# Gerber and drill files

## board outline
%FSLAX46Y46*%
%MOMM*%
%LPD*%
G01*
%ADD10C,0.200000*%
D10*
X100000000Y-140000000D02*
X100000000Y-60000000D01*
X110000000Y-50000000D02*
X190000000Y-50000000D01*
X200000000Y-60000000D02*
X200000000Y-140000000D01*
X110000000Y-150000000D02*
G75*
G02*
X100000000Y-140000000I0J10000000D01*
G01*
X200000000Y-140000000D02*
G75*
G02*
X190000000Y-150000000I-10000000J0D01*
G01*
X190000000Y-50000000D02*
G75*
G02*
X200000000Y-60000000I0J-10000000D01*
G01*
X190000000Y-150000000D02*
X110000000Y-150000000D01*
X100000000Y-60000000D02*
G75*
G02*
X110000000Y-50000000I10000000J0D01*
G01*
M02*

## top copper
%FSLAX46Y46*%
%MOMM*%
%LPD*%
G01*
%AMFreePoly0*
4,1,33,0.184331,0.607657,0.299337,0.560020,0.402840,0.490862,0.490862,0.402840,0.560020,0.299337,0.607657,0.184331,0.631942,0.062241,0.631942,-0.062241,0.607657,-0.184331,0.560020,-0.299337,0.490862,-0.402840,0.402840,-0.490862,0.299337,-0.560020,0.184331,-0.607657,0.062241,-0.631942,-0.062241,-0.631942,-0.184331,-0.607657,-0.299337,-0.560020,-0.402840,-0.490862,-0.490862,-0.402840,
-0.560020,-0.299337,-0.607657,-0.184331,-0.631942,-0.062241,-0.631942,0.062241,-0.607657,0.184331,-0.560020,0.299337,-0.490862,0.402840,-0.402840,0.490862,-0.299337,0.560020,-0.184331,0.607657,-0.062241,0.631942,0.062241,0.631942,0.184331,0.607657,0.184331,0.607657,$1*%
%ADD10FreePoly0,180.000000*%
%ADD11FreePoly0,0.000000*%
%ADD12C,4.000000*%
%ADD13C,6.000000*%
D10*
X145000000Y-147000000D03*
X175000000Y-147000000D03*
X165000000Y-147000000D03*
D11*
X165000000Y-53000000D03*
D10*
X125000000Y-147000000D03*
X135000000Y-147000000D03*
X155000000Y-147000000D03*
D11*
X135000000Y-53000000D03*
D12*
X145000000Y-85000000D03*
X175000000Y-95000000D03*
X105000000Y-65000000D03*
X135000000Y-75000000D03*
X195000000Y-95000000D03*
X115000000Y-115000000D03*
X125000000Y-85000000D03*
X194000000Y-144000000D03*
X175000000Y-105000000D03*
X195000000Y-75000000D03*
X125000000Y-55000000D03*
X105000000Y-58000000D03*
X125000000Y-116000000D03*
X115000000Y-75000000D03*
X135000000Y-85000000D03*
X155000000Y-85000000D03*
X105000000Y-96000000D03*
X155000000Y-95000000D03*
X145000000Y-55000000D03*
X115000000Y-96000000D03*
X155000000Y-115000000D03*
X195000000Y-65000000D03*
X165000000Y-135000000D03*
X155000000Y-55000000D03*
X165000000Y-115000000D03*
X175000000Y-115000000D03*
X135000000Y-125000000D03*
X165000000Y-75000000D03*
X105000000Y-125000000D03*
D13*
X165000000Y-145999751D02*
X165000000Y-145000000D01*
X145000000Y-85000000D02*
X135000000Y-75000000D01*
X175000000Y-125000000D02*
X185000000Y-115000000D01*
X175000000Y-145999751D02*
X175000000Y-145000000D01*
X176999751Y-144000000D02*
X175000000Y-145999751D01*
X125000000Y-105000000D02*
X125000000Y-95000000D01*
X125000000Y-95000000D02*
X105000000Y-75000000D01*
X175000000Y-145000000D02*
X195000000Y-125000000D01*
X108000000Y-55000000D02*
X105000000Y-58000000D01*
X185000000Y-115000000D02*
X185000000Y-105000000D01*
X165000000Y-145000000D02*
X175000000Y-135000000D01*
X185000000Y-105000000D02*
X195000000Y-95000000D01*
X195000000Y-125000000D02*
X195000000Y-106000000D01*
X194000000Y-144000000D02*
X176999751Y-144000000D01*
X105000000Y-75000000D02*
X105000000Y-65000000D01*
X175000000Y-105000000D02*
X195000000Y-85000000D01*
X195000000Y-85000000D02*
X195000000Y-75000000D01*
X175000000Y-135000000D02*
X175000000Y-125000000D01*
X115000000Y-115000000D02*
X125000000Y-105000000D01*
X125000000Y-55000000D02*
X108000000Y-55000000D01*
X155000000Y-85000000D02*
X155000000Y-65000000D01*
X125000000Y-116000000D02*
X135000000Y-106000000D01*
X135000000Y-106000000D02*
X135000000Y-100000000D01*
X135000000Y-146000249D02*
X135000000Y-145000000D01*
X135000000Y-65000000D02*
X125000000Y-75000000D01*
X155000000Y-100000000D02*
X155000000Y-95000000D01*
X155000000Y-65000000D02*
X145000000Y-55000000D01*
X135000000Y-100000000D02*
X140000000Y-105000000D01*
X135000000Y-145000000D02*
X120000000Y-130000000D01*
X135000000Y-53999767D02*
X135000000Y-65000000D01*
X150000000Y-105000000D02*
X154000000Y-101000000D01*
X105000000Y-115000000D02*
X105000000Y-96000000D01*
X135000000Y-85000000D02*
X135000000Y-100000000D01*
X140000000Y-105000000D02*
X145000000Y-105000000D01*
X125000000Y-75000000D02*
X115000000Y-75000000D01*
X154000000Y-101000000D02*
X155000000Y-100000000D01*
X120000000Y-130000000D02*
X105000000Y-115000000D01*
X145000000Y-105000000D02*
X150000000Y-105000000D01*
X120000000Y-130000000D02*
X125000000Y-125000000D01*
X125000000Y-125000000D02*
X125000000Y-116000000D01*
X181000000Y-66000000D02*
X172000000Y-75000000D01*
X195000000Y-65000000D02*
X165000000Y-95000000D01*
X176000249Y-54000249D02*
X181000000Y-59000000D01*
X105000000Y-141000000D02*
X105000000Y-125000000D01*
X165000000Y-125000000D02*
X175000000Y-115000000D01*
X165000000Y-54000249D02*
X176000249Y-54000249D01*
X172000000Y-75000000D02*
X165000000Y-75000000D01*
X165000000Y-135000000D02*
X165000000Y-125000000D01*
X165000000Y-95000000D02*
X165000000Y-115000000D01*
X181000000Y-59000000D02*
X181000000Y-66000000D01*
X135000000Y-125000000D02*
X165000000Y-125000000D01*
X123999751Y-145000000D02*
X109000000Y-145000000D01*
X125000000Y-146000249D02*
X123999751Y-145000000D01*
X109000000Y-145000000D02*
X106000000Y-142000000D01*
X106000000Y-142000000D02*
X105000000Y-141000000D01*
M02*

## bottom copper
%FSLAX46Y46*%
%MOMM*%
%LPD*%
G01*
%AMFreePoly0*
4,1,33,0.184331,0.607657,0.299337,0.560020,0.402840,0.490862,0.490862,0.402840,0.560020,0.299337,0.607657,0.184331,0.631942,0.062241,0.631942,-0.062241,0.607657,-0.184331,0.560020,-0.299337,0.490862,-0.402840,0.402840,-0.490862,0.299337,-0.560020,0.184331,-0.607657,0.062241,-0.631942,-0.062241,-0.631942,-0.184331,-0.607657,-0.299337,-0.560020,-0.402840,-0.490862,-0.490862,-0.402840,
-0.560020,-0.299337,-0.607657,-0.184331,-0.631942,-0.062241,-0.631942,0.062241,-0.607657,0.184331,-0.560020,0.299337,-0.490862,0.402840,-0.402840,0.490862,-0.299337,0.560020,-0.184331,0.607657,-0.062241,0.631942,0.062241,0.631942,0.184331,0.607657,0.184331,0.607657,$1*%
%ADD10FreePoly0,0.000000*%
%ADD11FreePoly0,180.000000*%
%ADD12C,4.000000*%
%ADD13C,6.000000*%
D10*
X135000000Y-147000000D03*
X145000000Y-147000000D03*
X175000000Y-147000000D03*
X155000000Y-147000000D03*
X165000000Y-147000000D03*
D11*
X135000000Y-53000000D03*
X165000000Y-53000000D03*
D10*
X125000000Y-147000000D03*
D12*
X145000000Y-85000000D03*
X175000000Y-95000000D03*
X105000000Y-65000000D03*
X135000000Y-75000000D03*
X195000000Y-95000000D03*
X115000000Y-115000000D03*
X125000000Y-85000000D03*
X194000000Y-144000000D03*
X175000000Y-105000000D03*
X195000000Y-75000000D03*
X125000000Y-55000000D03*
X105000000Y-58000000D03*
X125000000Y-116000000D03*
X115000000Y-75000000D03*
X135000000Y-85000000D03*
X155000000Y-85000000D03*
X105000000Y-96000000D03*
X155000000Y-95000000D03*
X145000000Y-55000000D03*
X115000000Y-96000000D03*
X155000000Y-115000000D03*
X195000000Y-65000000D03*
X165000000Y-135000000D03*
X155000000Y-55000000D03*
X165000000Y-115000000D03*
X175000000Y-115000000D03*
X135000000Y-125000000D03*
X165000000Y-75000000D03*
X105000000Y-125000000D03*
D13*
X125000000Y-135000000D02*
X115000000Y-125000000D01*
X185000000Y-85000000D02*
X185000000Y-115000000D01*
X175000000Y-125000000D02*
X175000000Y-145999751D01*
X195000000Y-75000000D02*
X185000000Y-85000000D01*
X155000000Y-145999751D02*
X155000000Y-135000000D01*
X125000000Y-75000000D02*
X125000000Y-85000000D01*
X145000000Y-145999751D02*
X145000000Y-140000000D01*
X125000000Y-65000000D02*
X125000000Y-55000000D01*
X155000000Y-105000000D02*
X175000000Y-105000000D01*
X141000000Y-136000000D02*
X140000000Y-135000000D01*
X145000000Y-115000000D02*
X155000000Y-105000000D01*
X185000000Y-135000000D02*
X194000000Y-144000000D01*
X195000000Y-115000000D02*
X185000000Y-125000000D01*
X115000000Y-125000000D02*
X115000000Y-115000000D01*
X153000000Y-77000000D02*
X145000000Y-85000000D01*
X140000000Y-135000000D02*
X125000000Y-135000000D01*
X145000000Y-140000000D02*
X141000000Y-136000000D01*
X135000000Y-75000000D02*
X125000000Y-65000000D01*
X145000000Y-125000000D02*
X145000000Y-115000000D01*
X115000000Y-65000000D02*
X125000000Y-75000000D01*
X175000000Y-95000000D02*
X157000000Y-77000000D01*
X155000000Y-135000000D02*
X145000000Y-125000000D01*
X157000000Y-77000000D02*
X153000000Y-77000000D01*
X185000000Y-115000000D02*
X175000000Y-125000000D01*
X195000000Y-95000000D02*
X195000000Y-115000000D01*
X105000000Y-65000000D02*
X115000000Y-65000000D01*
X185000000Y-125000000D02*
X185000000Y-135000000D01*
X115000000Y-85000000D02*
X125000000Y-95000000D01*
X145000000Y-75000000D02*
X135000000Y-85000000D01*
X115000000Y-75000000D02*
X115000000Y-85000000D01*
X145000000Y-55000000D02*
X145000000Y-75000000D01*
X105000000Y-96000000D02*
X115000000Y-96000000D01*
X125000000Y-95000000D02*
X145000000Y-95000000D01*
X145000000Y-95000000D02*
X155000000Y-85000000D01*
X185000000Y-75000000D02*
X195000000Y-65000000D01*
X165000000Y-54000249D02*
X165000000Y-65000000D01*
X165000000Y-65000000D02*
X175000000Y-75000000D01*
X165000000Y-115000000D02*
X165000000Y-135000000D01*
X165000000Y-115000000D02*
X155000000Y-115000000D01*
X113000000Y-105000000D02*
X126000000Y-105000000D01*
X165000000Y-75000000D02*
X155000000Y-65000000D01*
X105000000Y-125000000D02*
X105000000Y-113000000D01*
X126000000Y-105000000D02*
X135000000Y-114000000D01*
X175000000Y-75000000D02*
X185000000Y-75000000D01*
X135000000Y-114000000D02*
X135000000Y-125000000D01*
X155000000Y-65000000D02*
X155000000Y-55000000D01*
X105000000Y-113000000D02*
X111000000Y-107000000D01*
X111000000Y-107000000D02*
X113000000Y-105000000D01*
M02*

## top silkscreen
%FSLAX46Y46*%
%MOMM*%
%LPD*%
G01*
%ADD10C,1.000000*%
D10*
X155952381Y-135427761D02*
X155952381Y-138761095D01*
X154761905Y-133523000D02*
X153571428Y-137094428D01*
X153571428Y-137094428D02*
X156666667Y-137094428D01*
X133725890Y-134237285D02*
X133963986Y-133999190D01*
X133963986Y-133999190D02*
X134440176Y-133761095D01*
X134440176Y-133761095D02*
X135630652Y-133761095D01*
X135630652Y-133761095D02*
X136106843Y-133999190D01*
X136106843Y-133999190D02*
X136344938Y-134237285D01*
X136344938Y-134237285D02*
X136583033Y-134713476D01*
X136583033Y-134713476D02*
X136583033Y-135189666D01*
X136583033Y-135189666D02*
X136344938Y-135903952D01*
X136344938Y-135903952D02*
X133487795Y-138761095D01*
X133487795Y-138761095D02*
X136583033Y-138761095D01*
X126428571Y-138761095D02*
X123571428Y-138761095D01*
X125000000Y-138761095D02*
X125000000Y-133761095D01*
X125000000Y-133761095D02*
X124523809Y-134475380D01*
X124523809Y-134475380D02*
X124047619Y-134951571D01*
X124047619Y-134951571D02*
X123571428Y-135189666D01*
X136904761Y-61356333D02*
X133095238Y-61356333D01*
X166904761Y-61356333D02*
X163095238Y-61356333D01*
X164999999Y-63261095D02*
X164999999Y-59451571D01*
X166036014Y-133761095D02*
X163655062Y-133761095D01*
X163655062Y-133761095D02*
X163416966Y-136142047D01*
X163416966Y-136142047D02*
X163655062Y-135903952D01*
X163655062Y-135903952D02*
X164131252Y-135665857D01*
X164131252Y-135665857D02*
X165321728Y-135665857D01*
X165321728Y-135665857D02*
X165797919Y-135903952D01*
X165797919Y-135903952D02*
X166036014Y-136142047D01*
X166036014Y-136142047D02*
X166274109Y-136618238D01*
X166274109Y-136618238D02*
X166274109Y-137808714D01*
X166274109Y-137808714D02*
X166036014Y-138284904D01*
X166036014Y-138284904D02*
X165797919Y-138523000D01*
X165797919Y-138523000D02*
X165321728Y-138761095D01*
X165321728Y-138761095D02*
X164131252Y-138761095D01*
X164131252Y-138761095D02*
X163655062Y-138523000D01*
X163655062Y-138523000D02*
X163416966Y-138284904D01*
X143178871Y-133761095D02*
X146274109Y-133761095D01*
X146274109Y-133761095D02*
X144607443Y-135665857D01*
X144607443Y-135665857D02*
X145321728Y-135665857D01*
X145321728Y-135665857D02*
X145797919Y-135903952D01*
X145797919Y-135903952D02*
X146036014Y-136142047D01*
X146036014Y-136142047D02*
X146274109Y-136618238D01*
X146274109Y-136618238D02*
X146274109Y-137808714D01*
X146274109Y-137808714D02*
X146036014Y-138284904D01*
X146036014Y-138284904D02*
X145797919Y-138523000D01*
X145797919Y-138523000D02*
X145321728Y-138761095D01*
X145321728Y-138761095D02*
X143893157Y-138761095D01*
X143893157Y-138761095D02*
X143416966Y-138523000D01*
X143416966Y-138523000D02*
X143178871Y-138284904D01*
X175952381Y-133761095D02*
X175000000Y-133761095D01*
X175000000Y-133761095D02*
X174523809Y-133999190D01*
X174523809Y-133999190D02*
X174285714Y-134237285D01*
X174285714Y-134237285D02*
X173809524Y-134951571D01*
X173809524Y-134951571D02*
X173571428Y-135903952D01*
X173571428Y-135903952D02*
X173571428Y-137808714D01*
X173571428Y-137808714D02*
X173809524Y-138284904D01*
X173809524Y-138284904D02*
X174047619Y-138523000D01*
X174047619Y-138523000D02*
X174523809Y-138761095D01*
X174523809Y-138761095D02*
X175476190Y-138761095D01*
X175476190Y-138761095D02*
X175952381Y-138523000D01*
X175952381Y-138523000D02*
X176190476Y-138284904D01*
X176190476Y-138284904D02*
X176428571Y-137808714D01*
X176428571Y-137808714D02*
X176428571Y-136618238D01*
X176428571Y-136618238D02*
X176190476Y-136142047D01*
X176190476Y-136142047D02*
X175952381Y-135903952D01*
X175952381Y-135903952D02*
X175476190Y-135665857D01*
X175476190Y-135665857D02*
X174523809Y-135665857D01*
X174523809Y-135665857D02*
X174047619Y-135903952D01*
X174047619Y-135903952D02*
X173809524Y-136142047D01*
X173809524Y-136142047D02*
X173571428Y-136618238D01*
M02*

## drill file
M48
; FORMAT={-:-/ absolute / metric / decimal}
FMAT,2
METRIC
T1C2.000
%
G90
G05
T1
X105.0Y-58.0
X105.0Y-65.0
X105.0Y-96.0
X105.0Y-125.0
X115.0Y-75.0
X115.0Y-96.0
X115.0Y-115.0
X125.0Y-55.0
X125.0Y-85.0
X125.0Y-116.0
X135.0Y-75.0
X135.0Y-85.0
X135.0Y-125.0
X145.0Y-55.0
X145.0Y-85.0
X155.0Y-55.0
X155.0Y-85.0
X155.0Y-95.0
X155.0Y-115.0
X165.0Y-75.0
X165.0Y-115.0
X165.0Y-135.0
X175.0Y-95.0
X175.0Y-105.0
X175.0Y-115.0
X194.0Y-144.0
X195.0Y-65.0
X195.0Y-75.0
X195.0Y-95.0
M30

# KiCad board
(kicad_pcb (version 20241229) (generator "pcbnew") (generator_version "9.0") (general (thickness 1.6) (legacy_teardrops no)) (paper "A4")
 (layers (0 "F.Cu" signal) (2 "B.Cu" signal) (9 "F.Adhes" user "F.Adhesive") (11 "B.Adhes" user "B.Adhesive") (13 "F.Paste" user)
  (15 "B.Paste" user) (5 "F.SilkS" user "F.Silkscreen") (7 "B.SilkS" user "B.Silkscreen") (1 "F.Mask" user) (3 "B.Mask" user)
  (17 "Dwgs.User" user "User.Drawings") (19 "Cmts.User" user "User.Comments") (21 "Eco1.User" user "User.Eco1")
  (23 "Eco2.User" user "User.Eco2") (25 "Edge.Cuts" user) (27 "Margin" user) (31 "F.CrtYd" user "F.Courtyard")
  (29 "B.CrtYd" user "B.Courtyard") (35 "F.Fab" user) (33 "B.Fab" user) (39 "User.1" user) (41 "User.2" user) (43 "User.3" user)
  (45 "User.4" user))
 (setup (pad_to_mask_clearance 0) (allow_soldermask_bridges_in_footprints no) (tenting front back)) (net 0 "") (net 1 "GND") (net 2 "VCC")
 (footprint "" (layer "F.Cu") (at 145 147)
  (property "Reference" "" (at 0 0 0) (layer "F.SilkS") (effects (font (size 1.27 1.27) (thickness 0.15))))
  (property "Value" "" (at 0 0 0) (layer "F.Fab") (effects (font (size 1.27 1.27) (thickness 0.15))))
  (pad "1" smd custom (at 0 0 180) (size 1.27 1.27) (layers "F.Cu" "F.Mask" "F.Paste") (options (clearance outline) (anchor circle))
   (primitives)))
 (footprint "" (layer "F.Cu") (at 135 147)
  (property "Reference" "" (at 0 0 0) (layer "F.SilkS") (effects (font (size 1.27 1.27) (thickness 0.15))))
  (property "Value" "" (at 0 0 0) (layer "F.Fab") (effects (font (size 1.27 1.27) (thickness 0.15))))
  (pad "1" smd custom (at 0 0) (size 1.27 1.27) (layers "B.Cu" "B.Mask" "B.Paste") (options (clearance outline) (anchor circle))
   (primitives)))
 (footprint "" (layer "F.Cu") (at 175 147)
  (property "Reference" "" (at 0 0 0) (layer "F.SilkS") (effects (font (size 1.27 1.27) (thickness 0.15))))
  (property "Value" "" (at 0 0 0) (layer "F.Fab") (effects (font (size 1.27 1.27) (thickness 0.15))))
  (pad "1" smd custom (at 0 0 180) (size 1.27 1.27) (layers "F.Cu" "F.Mask" "F.Paste") (options (clearance outline) (anchor circle))
   (primitives)))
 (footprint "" (layer "F.Cu") (at 165 147)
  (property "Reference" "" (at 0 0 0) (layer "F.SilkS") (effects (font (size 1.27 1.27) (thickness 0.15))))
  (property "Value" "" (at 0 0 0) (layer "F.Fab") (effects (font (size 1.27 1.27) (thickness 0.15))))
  (pad "1" smd custom (at 0 0 180) (size 1.27 1.27) (layers "F.Cu" "F.Mask" "F.Paste") (options (clearance outline) (anchor circle))
   (primitives)))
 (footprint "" (layer "F.Cu") (at 145 147)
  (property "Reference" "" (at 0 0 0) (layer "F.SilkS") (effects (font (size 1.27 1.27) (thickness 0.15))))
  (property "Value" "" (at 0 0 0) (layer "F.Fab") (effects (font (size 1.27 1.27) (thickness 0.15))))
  (pad "1" smd custom (at 0 0) (size 1.27 1.27) (layers "B.Cu" "B.Mask" "B.Paste") (options (clearance outline) (anchor circle))
   (primitives)))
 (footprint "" (layer "F.Cu") (at 175 147)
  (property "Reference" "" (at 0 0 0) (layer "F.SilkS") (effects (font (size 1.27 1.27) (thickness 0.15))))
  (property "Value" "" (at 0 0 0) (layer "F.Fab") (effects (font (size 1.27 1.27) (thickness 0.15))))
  (pad "1" smd custom (at 0 0) (size 1.27 1.27) (layers "B.Cu" "B.Mask" "B.Paste") (options (clearance outline) (anchor circle))
   (primitives)))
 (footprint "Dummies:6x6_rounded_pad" (layer "F.Cu") (at 165 53)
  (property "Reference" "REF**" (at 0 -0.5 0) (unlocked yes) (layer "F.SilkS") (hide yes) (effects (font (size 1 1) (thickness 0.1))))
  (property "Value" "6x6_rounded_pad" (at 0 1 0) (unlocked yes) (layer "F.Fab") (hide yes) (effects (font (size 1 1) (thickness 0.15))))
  (pad "1" smd custom (at 0 0) (size 1.27 1.27) (layers "F.Cu" "F.Mask" "F.Paste") (options (clearance outline) (anchor circle))
   (primitives)))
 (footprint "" (layer "F.Cu") (at 155 147)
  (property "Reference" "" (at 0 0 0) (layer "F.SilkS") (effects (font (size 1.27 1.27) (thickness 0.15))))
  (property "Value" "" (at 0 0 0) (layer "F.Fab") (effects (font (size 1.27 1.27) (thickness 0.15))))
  (pad "1" smd custom (at 0 0) (size 1.27 1.27) (layers "B.Cu" "B.Mask" "B.Paste") (options (clearance outline) (anchor circle))
   (primitives)))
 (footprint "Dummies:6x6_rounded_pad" (layer "F.Cu") (at 125 147 180)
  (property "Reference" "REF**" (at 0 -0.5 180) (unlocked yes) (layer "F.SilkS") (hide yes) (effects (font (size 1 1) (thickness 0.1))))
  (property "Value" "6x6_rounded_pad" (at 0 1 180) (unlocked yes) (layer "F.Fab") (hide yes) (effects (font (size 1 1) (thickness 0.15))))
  (pad "1" smd custom (at 0 0 180) (size 1.27 1.27) (layers "F.Cu" "F.Mask" "F.Paste") (options (clearance outline) (anchor circle))
   (primitives)))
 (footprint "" (layer "F.Cu") (at 135 147)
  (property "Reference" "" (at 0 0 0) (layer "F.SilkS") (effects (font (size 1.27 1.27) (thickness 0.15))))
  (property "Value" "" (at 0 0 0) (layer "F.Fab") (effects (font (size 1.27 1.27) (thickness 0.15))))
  (pad "1" smd custom (at 0 0 180) (size 1.27 1.27) (layers "F.Cu" "F.Mask" "F.Paste") (options (clearance outline) (anchor circle))
   (primitives)))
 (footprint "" (layer "F.Cu") (at 165 147)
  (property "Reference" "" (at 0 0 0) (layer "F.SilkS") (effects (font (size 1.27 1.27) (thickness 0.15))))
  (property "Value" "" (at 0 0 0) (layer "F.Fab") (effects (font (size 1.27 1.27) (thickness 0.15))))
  (pad "1" smd custom (at 0 0) (size 1.27 1.27) (layers "B.Cu" "B.Mask" "B.Paste") (options (clearance outline) (anchor circle))
   (primitives)))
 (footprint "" (layer "F.Cu") (at 155 147)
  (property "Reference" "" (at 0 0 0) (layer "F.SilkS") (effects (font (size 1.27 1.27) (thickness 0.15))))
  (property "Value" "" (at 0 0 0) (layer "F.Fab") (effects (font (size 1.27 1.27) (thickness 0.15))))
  (pad "1" smd custom (at 0 0 180) (size 1.27 1.27) (layers "F.Cu" "F.Mask" "F.Paste") (options (clearance outline) (anchor circle))
   (primitives)))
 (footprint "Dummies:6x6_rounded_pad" (layer "F.Cu") (at 135 53)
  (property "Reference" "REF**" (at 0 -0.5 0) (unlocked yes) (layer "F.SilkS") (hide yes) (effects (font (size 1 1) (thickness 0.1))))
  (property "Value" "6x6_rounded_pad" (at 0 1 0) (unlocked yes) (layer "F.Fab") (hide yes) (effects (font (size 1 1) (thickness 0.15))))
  (pad "1" smd custom (at 0 0) (size 1.27 1.27) (layers "F.Cu" "F.Mask" "F.Paste") (options (clearance outline) (anchor circle))
   (primitives)))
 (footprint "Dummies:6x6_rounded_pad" (layer "B.Cu") (at 135 53 180)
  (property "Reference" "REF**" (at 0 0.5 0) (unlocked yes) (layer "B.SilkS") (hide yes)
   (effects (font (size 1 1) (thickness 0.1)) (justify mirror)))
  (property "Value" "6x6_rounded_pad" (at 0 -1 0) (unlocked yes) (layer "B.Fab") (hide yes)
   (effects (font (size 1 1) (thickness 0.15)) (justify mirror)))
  (pad "1" smd custom (at 0 0 180) (size 1.27 1.27) (layers "B.Cu" "B.Mask" "B.Paste") (options (clearance outline) (anchor circle))
   (primitives)))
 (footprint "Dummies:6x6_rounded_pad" (layer "B.Cu") (at 165 53 180)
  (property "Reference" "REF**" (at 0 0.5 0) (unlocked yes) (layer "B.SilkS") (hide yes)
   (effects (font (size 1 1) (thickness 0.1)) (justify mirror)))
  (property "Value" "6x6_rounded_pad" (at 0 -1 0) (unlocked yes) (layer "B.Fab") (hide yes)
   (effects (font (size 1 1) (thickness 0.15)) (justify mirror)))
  (pad "1" smd custom (at 0 0 180) (size 1.27 1.27) (layers "B.Cu" "B.Mask" "B.Paste") (options (clearance outline) (anchor circle))
   (primitives)))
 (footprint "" (layer "B.Cu") (at 125 147 180)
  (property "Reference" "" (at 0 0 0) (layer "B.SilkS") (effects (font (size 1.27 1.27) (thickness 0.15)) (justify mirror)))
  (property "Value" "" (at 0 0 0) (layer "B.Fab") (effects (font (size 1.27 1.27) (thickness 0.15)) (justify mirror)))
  (pad "1" smd custom (at 0 0) (size 1.27 1.27) (layers "B.Cu" "B.Mask" "B.Paste") (options (clearance outline) (anchor circle))
   (primitives)))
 (gr_line (start 100 140) (end 100 60) (stroke (width 0.2) (type default)) (layer "Edge.Cuts"))
 (gr_line (start 110 50) (end 190 50) (stroke (width 0.2) (type default)) (layer "Edge.Cuts"))
 (gr_line (start 200 60) (end 200 140) (stroke (width 0.2) (type default)) (layer "Edge.Cuts"))
 (gr_arc (start 110 150) (mid 102.928932 147.071068) (end 100 140) (stroke (width 0.2) (type default)) (layer "Edge.Cuts"))
 (gr_arc (start 200 140) (mid 197.071068 147.071068) (end 190 150) (stroke (width 0.2) (type default)) (layer "Edge.Cuts"))
 (gr_arc (start 190 50) (mid 197.071068 52.928932) (end 200 60) (stroke (width 0.2) (type default)) (layer "Edge.Cuts"))
 (gr_line (start 190 150) (end 110 150) (stroke (width 0.2) (type default)) (layer "Edge.Cuts"))
 (gr_arc (start 100 60) (mid 102.928932 52.928932) (end 110 50) (stroke (width 0.2) (type default)) (layer "Edge.Cuts"))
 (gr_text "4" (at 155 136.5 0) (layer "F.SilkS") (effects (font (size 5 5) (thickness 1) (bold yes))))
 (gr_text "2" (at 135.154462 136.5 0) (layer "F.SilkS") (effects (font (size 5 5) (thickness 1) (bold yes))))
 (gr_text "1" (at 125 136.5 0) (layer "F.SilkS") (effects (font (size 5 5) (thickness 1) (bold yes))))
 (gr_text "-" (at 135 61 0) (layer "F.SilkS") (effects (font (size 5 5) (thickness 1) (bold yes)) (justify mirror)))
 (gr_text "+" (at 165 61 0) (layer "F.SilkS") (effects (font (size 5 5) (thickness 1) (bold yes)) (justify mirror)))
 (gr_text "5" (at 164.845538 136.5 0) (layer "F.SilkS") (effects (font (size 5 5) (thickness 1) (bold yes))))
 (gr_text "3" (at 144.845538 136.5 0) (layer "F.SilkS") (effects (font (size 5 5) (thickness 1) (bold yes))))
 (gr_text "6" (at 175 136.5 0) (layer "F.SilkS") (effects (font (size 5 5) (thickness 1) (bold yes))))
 (segment (start 165 145.999751) (end 165 145) (width 6) (layer "F.Cu") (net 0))
 (segment (start 145 85) (end 135 75) (width 6) (layer "F.Cu") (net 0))
 (segment (start 175 125) (end 185 115) (width 6) (layer "F.Cu") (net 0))
 (segment (start 175 145.999751) (end 175 145) (width 6) (layer "F.Cu") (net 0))
 (segment (start 176.999751 144) (end 175 145.999751) (width 6) (layer "F.Cu") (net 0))
 (segment (start 125 105) (end 125 95) (width 6) (layer "F.Cu") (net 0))
 (segment (start 125 95) (end 105 75) (width 6) (layer "F.Cu") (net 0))
 (segment (start 175 145) (end 195 125) (width 6) (layer "F.Cu") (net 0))
 (segment (start 108 55) (end 105 58) (width 6) (layer "F.Cu") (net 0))
 (segment (start 185 115) (end 185 105) (width 6) (layer "F.Cu") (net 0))
 (segment (start 165 145) (end 175 135) (width 6) (layer "F.Cu") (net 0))
 (segment (start 185 105) (end 195 95) (width 6) (layer "F.Cu") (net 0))
 (segment (start 195 125) (end 195 106) (width 6) (layer "F.Cu") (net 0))
 (segment (start 194 144) (end 176.999751 144) (width 6) (layer "F.Cu") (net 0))
 (segment (start 105 75) (end 105 65) (width 6) (layer "F.Cu") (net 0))
 (segment (start 175 105) (end 195 85) (width 6) (layer "F.Cu") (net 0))
 (segment (start 195 85) (end 195 75) (width 6) (layer "F.Cu") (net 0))
 (segment (start 175 135) (end 175 125) (width 6) (layer "F.Cu") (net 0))
 (segment (start 115 115) (end 125 105) (width 6) (layer "F.Cu") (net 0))
 (segment (start 125 55) (end 108 55) (width 6) (layer "F.Cu") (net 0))
 (via (at 145 85) (size 4) (drill 2) (layers "F.Cu" "B.Cu") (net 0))
 (via (at 175 95) (size 4) (drill 2) (layers "F.Cu" "B.Cu") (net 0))
 (via (at 105 65) (size 4) (drill 2) (layers "F.Cu" "B.Cu") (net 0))
 (via (at 135 75) (size 4) (drill 2) (layers "F.Cu" "B.Cu") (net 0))
 (via (at 195 95) (size 4) (drill 2) (layers "F.Cu" "B.Cu") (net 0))
 (via (at 115 115) (size 4) (drill 2) (layers "F.Cu" "B.Cu") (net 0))
 (via (at 125 85) (size 4) (drill 2) (layers "F.Cu" "B.Cu") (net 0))
 (via (at 194 144) (size 4) (drill 2) (layers "F.Cu" "B.Cu") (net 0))
 (via (at 175 105) (size 4) (drill 2) (layers "F.Cu" "B.Cu") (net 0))
 (via (at 195 75) (size 4) (drill 2) (layers "F.Cu" "B.Cu") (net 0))
 (via (at 125 55) (size 4) (drill 2) (layers "F.Cu" "B.Cu") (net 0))
 (via (at 105 58) (size 4) (drill 2) (layers "F.Cu" "B.Cu") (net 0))
 (segment (start 125 135) (end 115 125) (width 6) (layer "B.Cu") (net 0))
 (segment (start 185 85) (end 185 115) (width 6) (layer "B.Cu") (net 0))
 (segment (start 175 125) (end 175 145.999751) (width 6) (layer "B.Cu") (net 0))
 (segment (start 195 75) (end 185 85) (width 6) (layer "B.Cu") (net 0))
 (segment (start 155 145.999751) (end 155 135) (width 6) (layer "B.Cu") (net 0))
 (segment (start 125 75) (end 125 85) (width 6) (layer "B.Cu") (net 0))
 (segment (start 145 145.999751) (end 145 140) (width 6) (layer "B.Cu") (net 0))
 (segment (start 125 65) (end 125 55) (width 6) (layer "B.Cu") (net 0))
 (segment (start 155 105) (end 175 105) (width 6) (layer "B.Cu") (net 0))
 (segment (start 141 136) (end 140 135) (width 6) (layer "B.Cu") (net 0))
 (segment (start 145 115) (end 155 105) (width 6) (layer "B.Cu") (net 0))
 (segment (start 185 135) (end 194 144) (width 6) (layer "B.Cu") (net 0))
 (segment (start 195 115) (end 185 125) (width 6) (layer "B.Cu") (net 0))
 (segment (start 115 125) (end 115 115) (width 6) (layer "B.Cu") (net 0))
 (segment (start 153 77) (end 145 85) (width 6) (layer "B.Cu") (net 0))
 (segment (start 140 135) (end 125 135) (width 6) (layer "B.Cu") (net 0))
 (segment (start 145 140) (end 141 136) (width 6) (layer "B.Cu") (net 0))
 (segment (start 135 75) (end 125 65) (width 6) (layer "B.Cu") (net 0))
 (segment (start 145 125) (end 145 115) (width 6) (layer "B.Cu") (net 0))
 (segment (start 115 65) (end 125 75) (width 6) (layer "B.Cu") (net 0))
 (segment (start 175 95) (end 157 77) (width 6) (layer "B.Cu") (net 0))
 (segment (start 155 135) (end 145 125) (width 6) (layer "B.Cu") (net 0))
 (segment (start 157 77) (end 153 77) (width 6) (layer "B.Cu") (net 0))
 (segment (start 185 115) (end 175 125) (width 6) (layer "B.Cu") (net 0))
 (segment (start 195 95) (end 195 115) (width 6) (layer "B.Cu") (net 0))
 (segment (start 105 65) (end 115 65) (width 6) (layer "B.Cu") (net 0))
 (segment (start 185 125) (end 185 135) (width 6) (layer "B.Cu") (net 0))
 (segment (start 155 85) (end 155 65) (width 6) (layer "F.Cu") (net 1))
 (segment (start 125 116) (end 135 106) (width 6) (layer "F.Cu") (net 1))
 (segment (start 135 106) (end 135 100) (width 6) (layer "F.Cu") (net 1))
 (segment (start 135 146.000249) (end 135 145) (width 6) (layer "F.Cu") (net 1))
 (segment (start 135 65) (end 125 75) (width 6) (layer "F.Cu") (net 1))
 (segment (start 155 100) (end 155 95) (width 6) (layer "F.Cu") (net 1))
 (segment (start 155 65) (end 145 55) (width 6) (layer "F.Cu") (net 1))
 (segment (start 135 100) (end 140 105) (width 6) (layer "F.Cu") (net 1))
 (segment (start 135 145) (end 120 130) (width 6) (layer "F.Cu") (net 1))
 (segment (start 135 53.999767) (end 135 65) (width 6) (layer "F.Cu") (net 1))
 (segment (start 150 105) (end 154 101) (width 6) (layer "F.Cu") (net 1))
 (segment (start 105 115) (end 105 96) (width 6) (layer "F.Cu") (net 1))
 (segment (start 135 85) (end 135 100) (width 6) (layer "F.Cu") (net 1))
 (segment (start 140 105) (end 145 105) (width 6) (layer "F.Cu") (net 1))
 (segment (start 125 75) (end 115 75) (width 6) (layer "F.Cu") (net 1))
 (segment (start 154 101) (end 155 100) (width 6) (layer "F.Cu") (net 1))
 (segment (start 120 130) (end 105 115) (width 6) (layer "F.Cu") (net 1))
 (segment (start 145 105) (end 150 105) (width 6) (layer "F.Cu") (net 1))
 (segment (start 120 130) (end 125 125) (width 6) (layer "F.Cu") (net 1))
 (segment (start 125 125) (end 125 116) (width 6) (layer "F.Cu") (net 1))
 (via (at 125 116) (size 4) (drill 2) (layers "F.Cu" "B.Cu") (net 1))
 (via (at 115 75) (size 4) (drill 2) (layers "F.Cu" "B.Cu") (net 1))
 (via (at 135 85) (size 4) (drill 2) (layers "F.Cu" "B.Cu") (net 1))
 (via (at 155 85) (size 4) (drill 2) (layers "F.Cu" "B.Cu") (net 1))
 (via (at 105 96) (size 4) (drill 2) (layers "F.Cu" "B.Cu") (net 1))
 (via (at 155 95) (size 4) (drill 2) (layers "F.Cu" "B.Cu") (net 1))
 (via (at 145 55) (size 4) (drill 2) (layers "F.Cu" "B.Cu") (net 1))
 (via (at 115 96) (size 4) (drill 2) (layers "F.Cu" "B.Cu") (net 1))
 (segment (start 115 85) (end 125 95) (width 6) (layer "B.Cu") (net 1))
 (segment (start 145 75) (end 135 85) (width 6) (layer "B.Cu") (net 1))
 (segment (start 115 75) (end 115 85) (width 6) (layer "B.Cu") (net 1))
 (segment (start 145 55) (end 145 75) (width 6) (layer "B.Cu") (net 1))
 (segment (start 105 96) (end 115 96) (width 6) (layer "B.Cu") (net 1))
 (segment (start 125 95) (end 145 95) (width 6) (layer "B.Cu") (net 1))
 (segment (start 145 95) (end 155 85) (width 6) (layer "B.Cu") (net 1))
 (segment (start 181 66) (end 172 75) (width 6) (layer "F.Cu") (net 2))
 (segment (start 195 65) (end 165 95) (width 6) (layer "F.Cu") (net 2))
 (segment (start 176.000249 54.000249) (end 181 59) (width 6) (layer "F.Cu") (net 2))
 (segment (start 105 141) (end 105 125) (width 6) (layer "F.Cu") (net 2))
 (segment (start 165 125) (end 175 115) (width 6) (layer "F.Cu") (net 2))
 (segment (start 165 54.000249) (end 176.000249 54.000249) (width 6) (layer "F.Cu") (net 2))
 (segment (start 172 75) (end 165 75) (width 6) (layer "F.Cu") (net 2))
 (segment (start 165 135) (end 165 125) (width 6) (layer "F.Cu") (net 2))
 (segment (start 165 95) (end 165 115) (width 6) (layer "F.Cu") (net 2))
 (segment (start 181 59) (end 181 66) (width 6) (layer "F.Cu") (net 2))
 (segment (start 135 125) (end 165 125) (width 6) (layer "F.Cu") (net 2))
 (segment (start 123.999751 145) (end 109 145) (width 6) (layer "F.Cu") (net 2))
 (segment (start 125 146.000249) (end 123.999751 145) (width 6) (layer "F.Cu") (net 2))
 (segment (start 109 145) (end 106 142) (width 6) (layer "F.Cu") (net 2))
 (segment (start 106 142) (end 105 141) (width 6) (layer "F.Cu") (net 2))
 (via (at 155 115) (size 4) (drill 2) (layers "F.Cu" "B.Cu") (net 2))
 (via (at 195 65) (size 4) (drill 2) (layers "F.Cu" "B.Cu") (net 2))
 (via (at 165 135) (size 4) (drill 2) (layers "F.Cu" "B.Cu") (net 2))
 (via (at 155 55) (size 4) (drill 2) (layers "F.Cu" "B.Cu") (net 2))
 (via (at 165 115) (size 4) (drill 2) (layers "F.Cu" "B.Cu") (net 2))
 (via (at 175 115) (size 4) (drill 2) (layers "F.Cu" "B.Cu") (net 2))
 (via (at 135 125) (size 4) (drill 2) (layers "F.Cu" "B.Cu") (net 2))
 (via (at 165 75) (size 4) (drill 2) (layers "F.Cu" "B.Cu") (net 2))
 (via (at 105 125) (size 4) (drill 2) (layers "F.Cu" "B.Cu") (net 2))
 (segment (start 185 75) (end 195 65) (width 6) (layer "B.Cu") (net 2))
 (segment (start 165 54.000249) (end 165 65) (width 6) (layer "B.Cu") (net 2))
 (segment (start 165 65) (end 175 75) (width 6) (layer "B.Cu") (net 2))
 (segment (start 165 115) (end 165 135) (width 6) (layer "B.Cu") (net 2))
 (segment (start 165 115) (end 155 115) (width 6) (layer "B.Cu") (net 2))
 (segment (start 113 105) (end 126 105) (width 6) (layer "B.Cu") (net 2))
 (segment (start 165 75) (end 155 65) (width 6) (layer "B.Cu") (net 2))
 (segment (start 105 125) (end 105 113) (width 6) (layer "B.Cu") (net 2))
 (segment (start 126 105) (end 135 114) (width 6) (layer "B.Cu") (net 2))
 (segment (start 175 75) (end 185 75) (width 6) (layer "B.Cu") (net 2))
 (segment (start 135 114) (end 135 125) (width 6) (layer "B.Cu") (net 2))
 (segment (start 155 65) (end 155 55) (width 6) (layer "B.Cu") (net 2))
 (segment (start 105 113) (end 111 107) (width 6) (layer "B.Cu") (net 2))
 (segment (start 111 107) (end 113 105) (width 6) (layer "B.Cu") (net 2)))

